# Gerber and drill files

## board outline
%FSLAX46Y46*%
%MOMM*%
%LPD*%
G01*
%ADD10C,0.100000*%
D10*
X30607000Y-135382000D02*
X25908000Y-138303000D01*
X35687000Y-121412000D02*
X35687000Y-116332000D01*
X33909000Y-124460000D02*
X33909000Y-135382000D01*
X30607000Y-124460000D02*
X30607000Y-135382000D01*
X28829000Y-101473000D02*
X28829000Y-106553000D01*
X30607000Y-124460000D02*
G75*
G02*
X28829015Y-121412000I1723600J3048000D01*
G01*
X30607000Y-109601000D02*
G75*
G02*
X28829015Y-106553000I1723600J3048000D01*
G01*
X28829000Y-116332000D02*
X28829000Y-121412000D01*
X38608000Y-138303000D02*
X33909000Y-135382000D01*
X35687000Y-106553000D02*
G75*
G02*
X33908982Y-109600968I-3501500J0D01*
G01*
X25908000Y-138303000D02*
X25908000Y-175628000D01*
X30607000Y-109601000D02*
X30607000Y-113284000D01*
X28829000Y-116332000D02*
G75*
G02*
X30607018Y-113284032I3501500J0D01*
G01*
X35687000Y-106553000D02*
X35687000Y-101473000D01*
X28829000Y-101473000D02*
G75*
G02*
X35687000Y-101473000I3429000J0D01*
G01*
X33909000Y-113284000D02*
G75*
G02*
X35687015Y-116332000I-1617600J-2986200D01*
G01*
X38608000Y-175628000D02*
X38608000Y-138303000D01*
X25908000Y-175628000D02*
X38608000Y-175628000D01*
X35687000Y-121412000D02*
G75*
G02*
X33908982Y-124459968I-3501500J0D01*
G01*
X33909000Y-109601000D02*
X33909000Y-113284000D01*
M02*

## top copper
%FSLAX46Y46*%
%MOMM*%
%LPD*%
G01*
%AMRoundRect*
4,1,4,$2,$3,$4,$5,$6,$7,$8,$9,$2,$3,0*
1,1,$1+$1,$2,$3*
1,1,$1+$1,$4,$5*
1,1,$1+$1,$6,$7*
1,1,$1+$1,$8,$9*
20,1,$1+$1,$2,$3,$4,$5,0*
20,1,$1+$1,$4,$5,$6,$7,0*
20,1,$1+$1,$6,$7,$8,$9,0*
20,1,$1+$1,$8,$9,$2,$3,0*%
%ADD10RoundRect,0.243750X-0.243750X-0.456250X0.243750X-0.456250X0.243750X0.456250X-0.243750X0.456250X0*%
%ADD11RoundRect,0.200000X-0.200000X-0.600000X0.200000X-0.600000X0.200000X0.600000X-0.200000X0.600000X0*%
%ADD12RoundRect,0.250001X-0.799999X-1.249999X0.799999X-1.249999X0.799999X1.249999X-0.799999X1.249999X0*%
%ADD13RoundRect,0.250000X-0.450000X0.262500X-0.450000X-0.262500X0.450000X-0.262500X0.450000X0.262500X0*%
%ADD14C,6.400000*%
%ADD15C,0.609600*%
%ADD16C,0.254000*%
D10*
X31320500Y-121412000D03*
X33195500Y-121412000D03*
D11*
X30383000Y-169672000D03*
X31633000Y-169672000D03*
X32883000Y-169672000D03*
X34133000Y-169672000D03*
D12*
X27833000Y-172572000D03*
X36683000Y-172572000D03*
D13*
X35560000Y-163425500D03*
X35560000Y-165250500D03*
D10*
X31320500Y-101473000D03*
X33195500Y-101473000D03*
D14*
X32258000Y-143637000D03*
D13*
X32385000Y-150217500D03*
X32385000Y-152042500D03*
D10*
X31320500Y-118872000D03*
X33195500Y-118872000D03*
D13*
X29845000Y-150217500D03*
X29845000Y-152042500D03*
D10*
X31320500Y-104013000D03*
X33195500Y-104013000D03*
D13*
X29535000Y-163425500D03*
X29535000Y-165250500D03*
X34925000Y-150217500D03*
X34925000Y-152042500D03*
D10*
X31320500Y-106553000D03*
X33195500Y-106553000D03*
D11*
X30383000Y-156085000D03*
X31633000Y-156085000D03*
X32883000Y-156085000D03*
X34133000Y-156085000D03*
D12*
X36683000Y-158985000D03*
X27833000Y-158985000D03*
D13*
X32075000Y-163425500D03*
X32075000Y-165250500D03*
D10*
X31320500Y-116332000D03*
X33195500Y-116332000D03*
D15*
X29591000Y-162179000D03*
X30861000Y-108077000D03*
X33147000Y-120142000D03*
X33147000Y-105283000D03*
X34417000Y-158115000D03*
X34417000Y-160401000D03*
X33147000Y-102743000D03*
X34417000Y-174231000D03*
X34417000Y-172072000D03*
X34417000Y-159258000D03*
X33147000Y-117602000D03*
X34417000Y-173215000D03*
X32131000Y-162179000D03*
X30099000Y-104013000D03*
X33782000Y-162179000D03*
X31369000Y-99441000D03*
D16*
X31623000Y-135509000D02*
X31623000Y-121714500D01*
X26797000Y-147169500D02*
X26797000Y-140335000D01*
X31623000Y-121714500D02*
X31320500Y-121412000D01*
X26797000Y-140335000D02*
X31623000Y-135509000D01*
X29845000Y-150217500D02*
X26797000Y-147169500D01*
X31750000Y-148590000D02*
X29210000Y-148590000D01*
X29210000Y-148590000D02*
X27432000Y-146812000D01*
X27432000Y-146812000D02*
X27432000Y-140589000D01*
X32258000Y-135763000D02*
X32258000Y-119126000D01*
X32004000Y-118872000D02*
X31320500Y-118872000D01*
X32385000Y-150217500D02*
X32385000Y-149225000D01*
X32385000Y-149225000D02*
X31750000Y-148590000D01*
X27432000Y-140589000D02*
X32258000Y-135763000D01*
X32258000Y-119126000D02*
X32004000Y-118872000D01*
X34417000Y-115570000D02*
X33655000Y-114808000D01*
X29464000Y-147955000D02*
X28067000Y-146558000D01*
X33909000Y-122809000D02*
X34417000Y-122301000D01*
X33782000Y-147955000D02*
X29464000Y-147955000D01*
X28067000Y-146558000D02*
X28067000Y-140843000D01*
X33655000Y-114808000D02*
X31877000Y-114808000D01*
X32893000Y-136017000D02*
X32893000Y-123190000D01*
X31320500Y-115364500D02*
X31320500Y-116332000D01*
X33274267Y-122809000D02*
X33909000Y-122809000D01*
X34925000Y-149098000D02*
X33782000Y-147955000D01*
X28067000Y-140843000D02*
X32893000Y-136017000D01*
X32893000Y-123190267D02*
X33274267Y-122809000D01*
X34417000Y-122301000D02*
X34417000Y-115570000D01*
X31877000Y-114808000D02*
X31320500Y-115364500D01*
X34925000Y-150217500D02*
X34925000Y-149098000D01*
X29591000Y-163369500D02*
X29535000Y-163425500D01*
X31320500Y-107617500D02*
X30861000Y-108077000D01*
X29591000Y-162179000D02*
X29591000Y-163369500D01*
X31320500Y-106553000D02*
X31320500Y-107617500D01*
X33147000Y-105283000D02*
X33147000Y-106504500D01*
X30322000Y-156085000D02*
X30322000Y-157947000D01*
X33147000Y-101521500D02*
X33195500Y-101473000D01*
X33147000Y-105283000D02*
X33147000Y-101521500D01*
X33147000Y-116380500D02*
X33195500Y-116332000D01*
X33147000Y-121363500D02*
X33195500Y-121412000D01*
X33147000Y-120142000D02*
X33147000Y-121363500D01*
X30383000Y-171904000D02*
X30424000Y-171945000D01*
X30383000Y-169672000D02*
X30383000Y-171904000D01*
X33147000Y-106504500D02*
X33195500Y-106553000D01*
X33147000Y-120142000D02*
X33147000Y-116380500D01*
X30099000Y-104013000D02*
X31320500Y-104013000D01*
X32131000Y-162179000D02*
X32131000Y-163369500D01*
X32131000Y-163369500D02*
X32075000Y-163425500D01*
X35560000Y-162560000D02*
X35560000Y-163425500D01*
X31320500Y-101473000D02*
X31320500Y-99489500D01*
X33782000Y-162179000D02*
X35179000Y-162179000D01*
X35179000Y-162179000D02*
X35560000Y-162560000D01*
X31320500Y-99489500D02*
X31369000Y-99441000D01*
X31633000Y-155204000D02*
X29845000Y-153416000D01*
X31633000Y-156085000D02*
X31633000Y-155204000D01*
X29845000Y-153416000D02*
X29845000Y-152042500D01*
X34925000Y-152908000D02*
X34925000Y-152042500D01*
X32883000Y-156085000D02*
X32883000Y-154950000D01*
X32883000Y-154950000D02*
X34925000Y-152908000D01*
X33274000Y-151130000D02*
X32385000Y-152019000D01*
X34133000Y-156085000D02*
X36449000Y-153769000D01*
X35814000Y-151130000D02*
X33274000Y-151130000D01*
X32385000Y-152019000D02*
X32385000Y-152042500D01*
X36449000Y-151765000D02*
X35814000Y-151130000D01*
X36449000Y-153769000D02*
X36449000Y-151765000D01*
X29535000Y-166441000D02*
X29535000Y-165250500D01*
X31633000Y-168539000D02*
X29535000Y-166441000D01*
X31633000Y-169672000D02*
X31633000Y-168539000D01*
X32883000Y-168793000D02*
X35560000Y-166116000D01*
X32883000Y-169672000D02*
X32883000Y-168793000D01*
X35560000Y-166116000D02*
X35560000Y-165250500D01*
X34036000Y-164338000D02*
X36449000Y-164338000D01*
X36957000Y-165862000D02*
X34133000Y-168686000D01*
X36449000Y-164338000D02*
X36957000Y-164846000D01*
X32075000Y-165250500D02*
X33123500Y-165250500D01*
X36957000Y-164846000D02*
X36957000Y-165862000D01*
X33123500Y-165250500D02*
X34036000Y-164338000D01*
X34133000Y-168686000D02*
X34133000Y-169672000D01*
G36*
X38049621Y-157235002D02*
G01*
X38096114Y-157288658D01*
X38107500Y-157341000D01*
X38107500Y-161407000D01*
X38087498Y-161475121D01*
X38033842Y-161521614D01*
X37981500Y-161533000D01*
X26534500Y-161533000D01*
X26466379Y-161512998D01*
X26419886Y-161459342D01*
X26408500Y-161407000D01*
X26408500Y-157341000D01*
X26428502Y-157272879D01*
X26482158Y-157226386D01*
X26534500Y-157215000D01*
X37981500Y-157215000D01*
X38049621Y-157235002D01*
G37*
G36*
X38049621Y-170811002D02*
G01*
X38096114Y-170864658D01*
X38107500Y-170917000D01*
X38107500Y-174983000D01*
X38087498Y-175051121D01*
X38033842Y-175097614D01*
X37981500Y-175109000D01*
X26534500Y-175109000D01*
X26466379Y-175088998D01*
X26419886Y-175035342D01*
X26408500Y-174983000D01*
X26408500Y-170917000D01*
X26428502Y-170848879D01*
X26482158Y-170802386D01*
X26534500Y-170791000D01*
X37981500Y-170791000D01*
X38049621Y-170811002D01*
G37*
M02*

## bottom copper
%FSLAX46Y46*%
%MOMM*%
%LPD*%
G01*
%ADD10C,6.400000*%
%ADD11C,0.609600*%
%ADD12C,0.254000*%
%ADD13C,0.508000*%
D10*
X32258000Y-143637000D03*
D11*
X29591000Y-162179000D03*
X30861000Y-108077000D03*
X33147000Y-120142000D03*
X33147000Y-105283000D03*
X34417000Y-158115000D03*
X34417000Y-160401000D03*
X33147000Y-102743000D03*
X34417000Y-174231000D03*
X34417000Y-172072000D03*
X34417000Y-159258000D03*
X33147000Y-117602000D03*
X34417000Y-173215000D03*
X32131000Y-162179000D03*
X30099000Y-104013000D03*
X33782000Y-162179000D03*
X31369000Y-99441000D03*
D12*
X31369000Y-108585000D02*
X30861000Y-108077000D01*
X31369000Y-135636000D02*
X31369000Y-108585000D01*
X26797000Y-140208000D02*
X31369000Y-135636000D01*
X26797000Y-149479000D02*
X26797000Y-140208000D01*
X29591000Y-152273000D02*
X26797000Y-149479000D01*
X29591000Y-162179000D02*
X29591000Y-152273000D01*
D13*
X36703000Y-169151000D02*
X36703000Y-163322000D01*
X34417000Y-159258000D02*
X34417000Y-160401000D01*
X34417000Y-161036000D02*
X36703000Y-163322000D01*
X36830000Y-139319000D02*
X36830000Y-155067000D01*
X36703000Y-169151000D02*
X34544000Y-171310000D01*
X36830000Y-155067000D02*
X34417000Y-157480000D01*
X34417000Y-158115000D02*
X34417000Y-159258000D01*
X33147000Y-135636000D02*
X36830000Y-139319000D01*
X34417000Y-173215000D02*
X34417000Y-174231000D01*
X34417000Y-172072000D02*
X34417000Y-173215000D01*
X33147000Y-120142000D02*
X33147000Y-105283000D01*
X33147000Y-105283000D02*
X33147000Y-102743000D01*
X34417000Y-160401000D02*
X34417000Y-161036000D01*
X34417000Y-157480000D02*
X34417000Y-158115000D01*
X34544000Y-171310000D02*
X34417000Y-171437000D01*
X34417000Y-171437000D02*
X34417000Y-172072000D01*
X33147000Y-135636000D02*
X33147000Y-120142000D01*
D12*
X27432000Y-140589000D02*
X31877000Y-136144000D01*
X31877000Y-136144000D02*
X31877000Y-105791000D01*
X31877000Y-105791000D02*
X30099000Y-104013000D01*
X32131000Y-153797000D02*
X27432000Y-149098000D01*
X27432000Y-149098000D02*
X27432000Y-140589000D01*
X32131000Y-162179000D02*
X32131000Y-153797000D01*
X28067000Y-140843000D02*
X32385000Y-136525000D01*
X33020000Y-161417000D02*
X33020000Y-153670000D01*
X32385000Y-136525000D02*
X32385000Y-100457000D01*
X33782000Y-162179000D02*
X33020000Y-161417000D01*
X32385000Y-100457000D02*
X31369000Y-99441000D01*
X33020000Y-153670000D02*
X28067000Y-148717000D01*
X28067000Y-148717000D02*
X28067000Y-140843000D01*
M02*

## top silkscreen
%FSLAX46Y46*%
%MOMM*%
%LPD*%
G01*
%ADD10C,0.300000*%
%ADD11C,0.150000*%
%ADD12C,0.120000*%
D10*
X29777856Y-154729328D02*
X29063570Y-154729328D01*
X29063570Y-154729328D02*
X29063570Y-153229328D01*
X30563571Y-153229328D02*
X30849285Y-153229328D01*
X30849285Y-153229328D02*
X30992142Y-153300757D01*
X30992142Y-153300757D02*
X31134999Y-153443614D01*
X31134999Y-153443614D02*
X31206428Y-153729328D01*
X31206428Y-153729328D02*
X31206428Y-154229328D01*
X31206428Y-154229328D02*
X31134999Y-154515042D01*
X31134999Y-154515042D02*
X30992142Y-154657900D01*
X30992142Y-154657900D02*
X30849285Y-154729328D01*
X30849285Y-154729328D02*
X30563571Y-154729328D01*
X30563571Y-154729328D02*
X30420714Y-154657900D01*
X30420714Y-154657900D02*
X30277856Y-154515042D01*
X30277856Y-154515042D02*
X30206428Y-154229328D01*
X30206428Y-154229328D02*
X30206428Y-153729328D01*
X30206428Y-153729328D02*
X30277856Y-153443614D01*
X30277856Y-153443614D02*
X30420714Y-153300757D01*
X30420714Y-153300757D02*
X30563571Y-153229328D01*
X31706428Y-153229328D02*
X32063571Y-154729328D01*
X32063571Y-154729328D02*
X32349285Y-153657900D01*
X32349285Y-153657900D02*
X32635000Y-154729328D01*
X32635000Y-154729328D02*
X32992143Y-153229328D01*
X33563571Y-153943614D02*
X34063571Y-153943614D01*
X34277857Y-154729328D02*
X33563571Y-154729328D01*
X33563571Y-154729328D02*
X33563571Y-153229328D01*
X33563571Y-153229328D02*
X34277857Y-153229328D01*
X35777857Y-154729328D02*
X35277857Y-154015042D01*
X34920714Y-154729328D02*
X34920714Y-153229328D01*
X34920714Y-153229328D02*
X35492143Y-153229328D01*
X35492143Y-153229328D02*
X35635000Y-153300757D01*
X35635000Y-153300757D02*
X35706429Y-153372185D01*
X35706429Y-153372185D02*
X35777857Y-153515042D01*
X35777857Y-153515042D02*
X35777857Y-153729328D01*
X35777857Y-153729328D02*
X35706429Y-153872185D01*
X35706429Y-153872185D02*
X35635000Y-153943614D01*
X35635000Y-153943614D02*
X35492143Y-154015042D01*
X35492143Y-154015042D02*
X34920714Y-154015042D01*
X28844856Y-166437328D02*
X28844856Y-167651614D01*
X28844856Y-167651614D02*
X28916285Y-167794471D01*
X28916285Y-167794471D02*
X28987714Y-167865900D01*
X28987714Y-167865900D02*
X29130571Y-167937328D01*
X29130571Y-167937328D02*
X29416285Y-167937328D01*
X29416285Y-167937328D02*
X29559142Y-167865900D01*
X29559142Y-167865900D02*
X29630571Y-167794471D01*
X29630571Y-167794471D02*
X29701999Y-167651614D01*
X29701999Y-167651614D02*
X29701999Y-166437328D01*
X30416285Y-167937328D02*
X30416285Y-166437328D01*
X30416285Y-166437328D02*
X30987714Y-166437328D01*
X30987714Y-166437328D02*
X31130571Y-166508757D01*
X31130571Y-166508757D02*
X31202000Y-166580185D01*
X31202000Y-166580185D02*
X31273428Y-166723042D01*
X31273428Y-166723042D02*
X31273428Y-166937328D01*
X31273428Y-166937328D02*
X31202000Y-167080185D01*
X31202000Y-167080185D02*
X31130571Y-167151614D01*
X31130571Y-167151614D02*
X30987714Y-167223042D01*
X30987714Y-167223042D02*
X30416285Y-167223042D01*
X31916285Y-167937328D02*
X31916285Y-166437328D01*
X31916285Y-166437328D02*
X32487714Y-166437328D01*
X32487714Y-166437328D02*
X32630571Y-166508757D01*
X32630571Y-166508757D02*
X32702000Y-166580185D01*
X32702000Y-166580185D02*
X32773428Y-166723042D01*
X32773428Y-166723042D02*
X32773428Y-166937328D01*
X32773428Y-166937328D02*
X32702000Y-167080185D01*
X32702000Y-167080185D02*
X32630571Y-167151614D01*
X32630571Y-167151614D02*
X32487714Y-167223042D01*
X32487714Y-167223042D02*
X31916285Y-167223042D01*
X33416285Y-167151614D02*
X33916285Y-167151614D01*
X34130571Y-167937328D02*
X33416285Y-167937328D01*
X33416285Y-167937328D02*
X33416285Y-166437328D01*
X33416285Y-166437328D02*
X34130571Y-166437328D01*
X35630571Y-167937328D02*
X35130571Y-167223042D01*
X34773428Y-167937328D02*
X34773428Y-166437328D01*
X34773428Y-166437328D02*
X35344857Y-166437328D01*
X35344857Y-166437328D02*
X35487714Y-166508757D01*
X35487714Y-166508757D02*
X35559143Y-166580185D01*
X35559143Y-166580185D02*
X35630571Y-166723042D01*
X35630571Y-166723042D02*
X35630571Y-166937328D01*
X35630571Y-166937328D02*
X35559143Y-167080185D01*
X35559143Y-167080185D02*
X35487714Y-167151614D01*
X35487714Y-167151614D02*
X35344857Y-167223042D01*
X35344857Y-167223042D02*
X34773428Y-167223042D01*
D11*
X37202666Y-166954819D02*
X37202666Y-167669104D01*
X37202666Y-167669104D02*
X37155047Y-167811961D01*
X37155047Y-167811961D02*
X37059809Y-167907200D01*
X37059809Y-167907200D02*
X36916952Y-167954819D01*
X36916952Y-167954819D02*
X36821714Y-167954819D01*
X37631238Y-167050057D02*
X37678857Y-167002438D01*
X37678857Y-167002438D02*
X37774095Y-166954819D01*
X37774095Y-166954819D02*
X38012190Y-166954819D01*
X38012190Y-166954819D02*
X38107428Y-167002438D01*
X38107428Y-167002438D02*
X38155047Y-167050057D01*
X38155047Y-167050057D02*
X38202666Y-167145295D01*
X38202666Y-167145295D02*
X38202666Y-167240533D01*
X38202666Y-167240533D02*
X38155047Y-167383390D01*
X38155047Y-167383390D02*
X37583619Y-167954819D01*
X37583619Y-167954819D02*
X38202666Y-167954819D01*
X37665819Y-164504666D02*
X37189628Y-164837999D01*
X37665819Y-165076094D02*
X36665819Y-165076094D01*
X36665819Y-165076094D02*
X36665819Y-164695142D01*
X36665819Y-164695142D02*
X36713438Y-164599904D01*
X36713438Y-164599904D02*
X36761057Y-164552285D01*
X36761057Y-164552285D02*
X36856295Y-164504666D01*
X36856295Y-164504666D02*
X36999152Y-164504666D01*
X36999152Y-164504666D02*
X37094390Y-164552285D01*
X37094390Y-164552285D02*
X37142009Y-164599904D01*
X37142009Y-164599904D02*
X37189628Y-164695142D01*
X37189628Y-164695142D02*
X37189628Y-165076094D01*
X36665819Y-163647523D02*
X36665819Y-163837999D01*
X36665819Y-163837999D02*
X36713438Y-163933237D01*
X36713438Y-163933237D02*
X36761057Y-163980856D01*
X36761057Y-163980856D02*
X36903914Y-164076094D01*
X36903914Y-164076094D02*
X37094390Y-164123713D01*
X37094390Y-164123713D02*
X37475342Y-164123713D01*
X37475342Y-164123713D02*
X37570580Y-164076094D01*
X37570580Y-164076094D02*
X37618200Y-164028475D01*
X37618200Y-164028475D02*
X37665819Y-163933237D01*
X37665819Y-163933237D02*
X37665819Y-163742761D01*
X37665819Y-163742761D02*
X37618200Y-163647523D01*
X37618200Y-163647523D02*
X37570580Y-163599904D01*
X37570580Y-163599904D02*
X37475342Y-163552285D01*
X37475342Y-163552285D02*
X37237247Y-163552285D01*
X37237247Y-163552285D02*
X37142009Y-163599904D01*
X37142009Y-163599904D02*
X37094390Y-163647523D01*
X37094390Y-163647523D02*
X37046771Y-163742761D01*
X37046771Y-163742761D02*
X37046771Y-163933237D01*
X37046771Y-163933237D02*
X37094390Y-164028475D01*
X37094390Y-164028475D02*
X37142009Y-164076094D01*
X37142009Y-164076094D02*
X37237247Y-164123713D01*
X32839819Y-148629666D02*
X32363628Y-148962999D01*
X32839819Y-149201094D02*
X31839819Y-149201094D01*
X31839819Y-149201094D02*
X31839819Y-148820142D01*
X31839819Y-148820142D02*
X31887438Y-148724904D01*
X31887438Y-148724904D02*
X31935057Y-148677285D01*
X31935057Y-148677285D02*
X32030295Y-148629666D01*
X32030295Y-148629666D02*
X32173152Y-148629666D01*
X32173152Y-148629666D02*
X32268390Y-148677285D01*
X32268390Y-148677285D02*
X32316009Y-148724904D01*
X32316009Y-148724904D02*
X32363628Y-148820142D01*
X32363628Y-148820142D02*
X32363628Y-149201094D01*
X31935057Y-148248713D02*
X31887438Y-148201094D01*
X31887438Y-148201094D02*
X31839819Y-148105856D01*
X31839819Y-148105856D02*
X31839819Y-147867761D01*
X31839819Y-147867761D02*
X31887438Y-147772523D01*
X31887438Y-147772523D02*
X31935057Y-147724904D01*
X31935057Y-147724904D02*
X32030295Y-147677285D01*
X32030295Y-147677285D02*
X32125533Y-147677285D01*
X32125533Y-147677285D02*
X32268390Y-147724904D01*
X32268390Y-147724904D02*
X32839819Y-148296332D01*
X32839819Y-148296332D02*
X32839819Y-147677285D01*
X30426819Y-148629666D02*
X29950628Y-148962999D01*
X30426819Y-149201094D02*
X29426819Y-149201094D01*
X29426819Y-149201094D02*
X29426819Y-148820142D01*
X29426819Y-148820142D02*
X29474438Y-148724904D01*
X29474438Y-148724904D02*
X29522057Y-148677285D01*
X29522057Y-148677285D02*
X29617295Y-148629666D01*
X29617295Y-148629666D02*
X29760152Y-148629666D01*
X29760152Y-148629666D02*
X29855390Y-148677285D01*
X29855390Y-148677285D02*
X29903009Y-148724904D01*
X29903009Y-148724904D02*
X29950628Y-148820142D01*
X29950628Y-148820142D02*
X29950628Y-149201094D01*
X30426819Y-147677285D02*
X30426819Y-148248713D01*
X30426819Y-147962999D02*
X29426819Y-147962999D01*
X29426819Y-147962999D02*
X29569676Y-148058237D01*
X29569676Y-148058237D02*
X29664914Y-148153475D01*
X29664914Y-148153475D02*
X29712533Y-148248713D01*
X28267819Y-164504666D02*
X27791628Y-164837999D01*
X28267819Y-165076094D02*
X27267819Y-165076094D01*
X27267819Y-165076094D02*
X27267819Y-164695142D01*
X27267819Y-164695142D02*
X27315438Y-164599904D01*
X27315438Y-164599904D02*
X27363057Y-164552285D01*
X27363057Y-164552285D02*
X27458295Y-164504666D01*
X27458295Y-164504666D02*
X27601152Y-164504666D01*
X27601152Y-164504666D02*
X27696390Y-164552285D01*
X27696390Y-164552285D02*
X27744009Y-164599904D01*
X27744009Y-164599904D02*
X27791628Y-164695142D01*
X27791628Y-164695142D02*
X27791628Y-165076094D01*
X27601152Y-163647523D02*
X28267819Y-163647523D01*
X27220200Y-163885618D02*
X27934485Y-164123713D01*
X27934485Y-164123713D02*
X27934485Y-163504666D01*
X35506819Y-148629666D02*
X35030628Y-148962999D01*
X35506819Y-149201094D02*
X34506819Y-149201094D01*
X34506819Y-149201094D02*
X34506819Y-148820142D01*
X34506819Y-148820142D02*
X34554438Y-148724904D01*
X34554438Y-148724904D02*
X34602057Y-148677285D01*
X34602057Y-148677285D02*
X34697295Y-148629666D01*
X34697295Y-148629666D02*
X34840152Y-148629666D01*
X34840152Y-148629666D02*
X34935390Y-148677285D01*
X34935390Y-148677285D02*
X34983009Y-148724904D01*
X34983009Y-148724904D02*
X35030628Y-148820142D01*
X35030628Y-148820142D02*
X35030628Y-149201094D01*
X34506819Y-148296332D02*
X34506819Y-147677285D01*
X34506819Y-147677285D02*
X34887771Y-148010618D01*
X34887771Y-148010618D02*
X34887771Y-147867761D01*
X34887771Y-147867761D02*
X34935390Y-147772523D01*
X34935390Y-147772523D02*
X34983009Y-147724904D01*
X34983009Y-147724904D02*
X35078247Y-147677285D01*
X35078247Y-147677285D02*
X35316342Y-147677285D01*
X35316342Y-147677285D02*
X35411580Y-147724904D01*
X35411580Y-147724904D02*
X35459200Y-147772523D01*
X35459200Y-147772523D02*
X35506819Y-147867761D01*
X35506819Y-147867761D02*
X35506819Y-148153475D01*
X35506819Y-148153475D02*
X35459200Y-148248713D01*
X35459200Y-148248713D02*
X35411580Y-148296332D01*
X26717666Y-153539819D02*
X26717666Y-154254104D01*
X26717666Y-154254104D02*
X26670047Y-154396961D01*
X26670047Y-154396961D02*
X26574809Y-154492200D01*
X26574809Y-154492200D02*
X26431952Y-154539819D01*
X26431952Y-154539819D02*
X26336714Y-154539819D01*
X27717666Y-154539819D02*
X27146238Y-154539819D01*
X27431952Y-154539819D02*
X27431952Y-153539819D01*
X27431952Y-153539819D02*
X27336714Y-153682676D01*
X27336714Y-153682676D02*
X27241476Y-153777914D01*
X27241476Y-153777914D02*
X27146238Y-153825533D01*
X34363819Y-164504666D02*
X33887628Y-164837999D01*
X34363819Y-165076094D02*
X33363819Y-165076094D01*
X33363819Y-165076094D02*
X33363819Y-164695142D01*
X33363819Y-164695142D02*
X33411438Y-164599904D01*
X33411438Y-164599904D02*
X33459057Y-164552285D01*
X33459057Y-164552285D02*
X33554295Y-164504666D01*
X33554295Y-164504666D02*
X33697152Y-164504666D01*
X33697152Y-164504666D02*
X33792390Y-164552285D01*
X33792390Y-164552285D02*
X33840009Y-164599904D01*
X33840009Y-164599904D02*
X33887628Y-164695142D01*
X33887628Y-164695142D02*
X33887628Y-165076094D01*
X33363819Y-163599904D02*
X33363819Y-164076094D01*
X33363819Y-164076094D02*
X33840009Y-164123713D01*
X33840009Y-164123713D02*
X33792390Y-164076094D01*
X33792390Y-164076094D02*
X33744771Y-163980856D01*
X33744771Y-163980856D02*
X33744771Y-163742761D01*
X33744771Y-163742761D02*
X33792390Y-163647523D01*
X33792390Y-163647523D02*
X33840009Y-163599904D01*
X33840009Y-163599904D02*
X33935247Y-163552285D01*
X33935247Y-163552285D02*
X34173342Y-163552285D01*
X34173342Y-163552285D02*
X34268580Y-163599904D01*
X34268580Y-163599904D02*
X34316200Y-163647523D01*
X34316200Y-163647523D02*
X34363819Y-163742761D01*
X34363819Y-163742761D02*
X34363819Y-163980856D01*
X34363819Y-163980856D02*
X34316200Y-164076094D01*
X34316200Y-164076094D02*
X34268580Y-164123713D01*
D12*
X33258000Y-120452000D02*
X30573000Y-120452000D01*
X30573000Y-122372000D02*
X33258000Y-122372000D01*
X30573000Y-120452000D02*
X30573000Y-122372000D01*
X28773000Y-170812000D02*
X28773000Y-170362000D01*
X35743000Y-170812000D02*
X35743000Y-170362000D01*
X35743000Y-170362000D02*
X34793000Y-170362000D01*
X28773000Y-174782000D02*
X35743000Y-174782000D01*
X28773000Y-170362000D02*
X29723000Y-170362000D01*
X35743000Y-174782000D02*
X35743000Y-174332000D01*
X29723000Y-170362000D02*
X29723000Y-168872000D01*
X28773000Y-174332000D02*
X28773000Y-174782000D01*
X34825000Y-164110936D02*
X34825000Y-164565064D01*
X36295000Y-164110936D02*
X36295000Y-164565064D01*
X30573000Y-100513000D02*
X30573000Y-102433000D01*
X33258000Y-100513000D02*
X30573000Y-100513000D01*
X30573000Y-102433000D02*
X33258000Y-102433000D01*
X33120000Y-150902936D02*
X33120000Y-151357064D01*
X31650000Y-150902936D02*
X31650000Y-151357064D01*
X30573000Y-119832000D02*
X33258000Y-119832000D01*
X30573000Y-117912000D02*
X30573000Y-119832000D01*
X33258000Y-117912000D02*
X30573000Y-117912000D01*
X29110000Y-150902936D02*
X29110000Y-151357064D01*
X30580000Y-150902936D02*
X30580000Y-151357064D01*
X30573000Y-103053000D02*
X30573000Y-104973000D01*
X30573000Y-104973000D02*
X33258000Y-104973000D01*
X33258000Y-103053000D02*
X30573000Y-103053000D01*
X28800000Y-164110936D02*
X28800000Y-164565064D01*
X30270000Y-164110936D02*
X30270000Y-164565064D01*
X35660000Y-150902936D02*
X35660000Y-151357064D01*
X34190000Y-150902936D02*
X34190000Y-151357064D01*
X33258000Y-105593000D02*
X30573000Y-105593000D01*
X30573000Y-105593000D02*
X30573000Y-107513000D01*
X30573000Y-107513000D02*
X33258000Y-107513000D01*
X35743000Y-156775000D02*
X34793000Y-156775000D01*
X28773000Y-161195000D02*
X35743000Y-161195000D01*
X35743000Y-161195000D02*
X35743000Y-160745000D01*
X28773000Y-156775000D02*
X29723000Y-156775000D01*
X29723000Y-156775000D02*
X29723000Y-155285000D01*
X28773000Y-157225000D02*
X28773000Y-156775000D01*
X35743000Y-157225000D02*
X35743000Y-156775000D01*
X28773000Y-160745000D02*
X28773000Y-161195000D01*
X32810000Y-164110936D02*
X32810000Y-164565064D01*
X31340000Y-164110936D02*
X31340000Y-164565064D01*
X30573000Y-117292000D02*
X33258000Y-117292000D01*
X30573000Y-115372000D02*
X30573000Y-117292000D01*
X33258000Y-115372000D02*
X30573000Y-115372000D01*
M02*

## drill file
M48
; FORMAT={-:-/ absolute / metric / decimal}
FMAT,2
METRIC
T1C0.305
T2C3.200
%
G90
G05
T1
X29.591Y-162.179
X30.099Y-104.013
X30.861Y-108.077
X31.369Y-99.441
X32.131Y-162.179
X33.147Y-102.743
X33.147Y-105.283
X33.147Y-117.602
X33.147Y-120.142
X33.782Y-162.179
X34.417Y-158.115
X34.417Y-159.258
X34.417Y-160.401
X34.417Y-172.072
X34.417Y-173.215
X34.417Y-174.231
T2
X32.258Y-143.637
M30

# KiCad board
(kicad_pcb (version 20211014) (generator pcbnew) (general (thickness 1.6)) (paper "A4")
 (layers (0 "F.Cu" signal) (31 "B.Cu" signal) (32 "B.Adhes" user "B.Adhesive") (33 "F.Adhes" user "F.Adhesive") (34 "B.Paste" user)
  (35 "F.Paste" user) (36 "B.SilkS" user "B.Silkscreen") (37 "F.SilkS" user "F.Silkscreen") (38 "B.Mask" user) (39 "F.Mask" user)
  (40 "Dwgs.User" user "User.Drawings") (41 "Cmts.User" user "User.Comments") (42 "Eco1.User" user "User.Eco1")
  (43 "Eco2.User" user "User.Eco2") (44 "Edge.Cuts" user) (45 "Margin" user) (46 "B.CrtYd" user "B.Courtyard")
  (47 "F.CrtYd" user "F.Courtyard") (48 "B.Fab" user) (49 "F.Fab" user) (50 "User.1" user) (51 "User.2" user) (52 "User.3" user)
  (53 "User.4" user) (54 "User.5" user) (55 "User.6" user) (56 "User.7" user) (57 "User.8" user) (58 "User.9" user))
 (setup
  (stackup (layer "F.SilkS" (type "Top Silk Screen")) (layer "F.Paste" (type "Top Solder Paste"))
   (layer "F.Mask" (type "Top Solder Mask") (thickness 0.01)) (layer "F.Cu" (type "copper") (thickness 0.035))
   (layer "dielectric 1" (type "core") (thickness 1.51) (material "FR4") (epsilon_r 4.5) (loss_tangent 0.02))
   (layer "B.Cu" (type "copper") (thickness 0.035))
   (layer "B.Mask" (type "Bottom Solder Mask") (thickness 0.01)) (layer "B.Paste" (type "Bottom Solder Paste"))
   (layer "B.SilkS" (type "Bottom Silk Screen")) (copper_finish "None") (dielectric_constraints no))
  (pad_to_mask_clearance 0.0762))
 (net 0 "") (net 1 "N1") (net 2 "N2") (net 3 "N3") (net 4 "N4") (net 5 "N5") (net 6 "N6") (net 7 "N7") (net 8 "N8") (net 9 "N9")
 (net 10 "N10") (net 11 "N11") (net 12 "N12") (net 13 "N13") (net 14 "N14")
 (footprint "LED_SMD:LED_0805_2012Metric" (layer "F.Cu") (at 32.258 121.412)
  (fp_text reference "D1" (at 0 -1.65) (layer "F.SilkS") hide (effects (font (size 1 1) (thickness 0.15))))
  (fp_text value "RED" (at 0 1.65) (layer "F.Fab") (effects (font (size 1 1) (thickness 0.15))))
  (fp_line (start 1 -0.96) (end -1.685 -0.96) (layer "F.SilkS") (width 0.12))
  (fp_line (start -1.685 0.96) (end 1 0.96) (layer "F.SilkS") (width 0.12))
  (fp_line (start -1.685 -0.96) (end -1.685 0.96) (layer "F.SilkS") (width 0.12))
  (pad "1" smd roundrect (at -0.9375 0) (size 0.975 1.4) (layers "F.Cu" "F.Paste" "F.Mask") (roundrect_rratio 0.25) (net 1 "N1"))
  (pad "2" smd roundrect (at 0.9375 0) (size 0.975 1.4) (layers "F.Cu" "F.Paste" "F.Mask") (roundrect_rratio 0.25) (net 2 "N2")))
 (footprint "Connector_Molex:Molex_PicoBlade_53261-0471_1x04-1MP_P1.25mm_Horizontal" (layer "F.Cu") (at 32.258 172.072)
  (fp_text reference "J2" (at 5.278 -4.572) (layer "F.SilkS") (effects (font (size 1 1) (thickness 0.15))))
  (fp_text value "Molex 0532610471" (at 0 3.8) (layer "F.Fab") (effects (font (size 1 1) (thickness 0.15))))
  (fp_line (start -3.485 -1.26) (end -3.485 -1.71) (layer "F.SilkS") (width 0.12))
  (fp_line (start 3.485 -1.26) (end 3.485 -1.71) (layer "F.SilkS") (width 0.12))
  (fp_line (start 3.485 -1.71) (end 2.535 -1.71) (layer "F.SilkS") (width 0.12))
  (fp_line (start -3.485 2.71) (end 3.485 2.71) (layer "F.SilkS") (width 0.12))
  (fp_line (start -3.485 -1.71) (end -2.535 -1.71) (layer "F.SilkS") (width 0.12))
  (fp_line (start 3.485 2.71) (end 3.485 2.26) (layer "F.SilkS") (width 0.12))
  (fp_line (start -2.535 -1.71) (end -2.535 -3.2) (layer "F.SilkS") (width 0.12))
  (fp_line (start -3.485 2.26) (end -3.485 2.71) (layer "F.SilkS") (width 0.12))
  (pad "1" smd roundrect (at -1.875 -2.4) (size 0.8 1.6) (layers "F.Cu" "F.Paste" "F.Mask") (roundrect_rratio 0.25) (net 2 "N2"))
  (pad "2" smd roundrect (at -0.625 -2.4) (size 0.8 1.6) (layers "F.Cu" "F.Paste" "F.Mask") (roundrect_rratio 0.25) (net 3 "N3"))
  (pad "3" smd roundrect (at 0.625 -2.4) (size 0.8 1.6) (layers "F.Cu" "F.Paste" "F.Mask") (roundrect_rratio 0.25) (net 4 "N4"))
  (pad "4" smd roundrect (at 1.875 -2.4) (size 0.8 1.6) (layers "F.Cu" "F.Paste" "F.Mask") (roundrect_rratio 0.25) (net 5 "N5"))
  (pad "MP" smd roundrect (at -4.425 0.5) (size 2.1 3) (layers "F.Cu" "F.Paste" "F.Mask") (roundrect_rratio 0.119048) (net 2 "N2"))
  (pad "MP" smd roundrect (at 4.425 0.5) (size 2.1 3) (layers "F.Cu" "F.Paste" "F.Mask") (roundrect_rratio 0.119048) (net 2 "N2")))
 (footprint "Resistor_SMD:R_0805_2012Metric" (layer "F.Cu") (at 35.56 164.338 -90)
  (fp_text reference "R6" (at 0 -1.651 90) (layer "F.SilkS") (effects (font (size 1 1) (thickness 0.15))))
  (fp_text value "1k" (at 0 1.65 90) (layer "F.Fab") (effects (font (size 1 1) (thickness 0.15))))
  (fp_line (start -0.227064 0.735) (end 0.227064 0.735) (layer "F.SilkS") (width 0.12))
  (fp_line (start -0.227064 -0.735) (end 0.227064 -0.735) (layer "F.SilkS") (width 0.12))
  (pad "1" smd roundrect (at -0.9125 0 270) (size 1.025 1.4) (layers "F.Cu" "F.Paste" "F.Mask") (roundrect_rratio 0.243902) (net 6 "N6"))
  (pad "2" smd roundrect (at 0.9125 0 270) (size 1.025 1.4) (layers "F.Cu" "F.Paste" "F.Mask") (roundrect_rratio 0.243902) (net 4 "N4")))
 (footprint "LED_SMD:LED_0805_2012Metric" (layer "F.Cu") (at 32.258 101.473)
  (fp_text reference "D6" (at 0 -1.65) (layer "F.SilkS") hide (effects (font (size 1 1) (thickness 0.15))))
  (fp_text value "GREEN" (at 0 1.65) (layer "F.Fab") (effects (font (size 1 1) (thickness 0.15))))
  (fp_line (start -1.685 -0.96) (end -1.685 0.96) (layer "F.SilkS") (width 0.12))
  (fp_line (start 1 -0.96) (end -1.685 -0.96) (layer "F.SilkS") (width 0.12))
  (fp_line (start -1.685 0.96) (end 1 0.96) (layer "F.SilkS") (width 0.12))
  (pad "1" smd roundrect (at -0.9375 0) (size 0.975 1.4) (layers "F.Cu" "F.Paste" "F.Mask") (roundrect_rratio 0.25) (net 6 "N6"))
  (pad "2" smd roundrect (at 0.9375 0) (size 0.975 1.4) (layers "F.Cu" "F.Paste" "F.Mask") (roundrect_rratio 0.25) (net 2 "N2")))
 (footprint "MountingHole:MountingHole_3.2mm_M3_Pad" (layer "F.Cu") (at 32.258 143.637) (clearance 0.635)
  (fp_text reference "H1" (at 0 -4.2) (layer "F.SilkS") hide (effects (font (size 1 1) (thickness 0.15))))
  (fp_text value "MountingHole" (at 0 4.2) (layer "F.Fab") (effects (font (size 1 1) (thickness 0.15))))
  (pad "1" thru_hole circle (at 0 0) (size 6.4 6.4) (drill 3.2) (layers *.Cu *.Mask) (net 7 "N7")))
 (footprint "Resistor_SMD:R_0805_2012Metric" (layer "F.Cu") (at 32.385 151.13 -90)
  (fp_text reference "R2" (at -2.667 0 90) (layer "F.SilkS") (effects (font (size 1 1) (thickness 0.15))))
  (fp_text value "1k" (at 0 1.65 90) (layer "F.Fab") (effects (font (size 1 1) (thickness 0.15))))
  (fp_line (start -0.227064 -0.735) (end 0.227064 -0.735) (layer "F.SilkS") (width 0.12))
  (fp_line (start -0.227064 0.735) (end 0.227064 0.735) (layer "F.SilkS") (width 0.12))
  (pad "1" smd roundrect (at -0.9125 0 270) (size 1.025 1.4) (layers "F.Cu" "F.Paste" "F.Mask") (roundrect_rratio 0.243902) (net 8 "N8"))
  (pad "2" smd roundrect (at 0.9125 0 270) (size 1.025 1.4) (layers "F.Cu" "F.Paste" "F.Mask") (roundrect_rratio 0.243902) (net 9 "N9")))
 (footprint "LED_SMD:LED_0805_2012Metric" (layer "F.Cu") (at 32.258 118.872)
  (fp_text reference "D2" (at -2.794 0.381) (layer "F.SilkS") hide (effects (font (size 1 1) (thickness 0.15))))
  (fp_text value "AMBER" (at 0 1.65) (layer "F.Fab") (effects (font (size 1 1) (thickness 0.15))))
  (fp_line (start -1.685 0.96) (end 1 0.96) (layer "F.SilkS") (width 0.12))
  (fp_line (start -1.685 -0.96) (end -1.685 0.96) (layer "F.SilkS") (width 0.12))
  (fp_line (start 1 -0.96) (end -1.685 -0.96) (layer "F.SilkS") (width 0.12))
  (pad "1" smd roundrect (at -0.9375 0) (size 0.975 1.4) (layers "F.Cu" "F.Paste" "F.Mask") (roundrect_rratio 0.25) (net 8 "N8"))
  (pad "2" smd roundrect (at 0.9375 0) (size 0.975 1.4) (layers "F.Cu" "F.Paste" "F.Mask") (roundrect_rratio 0.25) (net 2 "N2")))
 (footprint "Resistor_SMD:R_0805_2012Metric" (layer "F.Cu") (at 29.845 151.13 -90)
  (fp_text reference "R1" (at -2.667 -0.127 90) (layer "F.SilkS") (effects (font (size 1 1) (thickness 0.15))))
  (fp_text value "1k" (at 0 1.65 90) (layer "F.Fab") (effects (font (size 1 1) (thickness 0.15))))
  (fp_line (start -0.227064 0.735) (end 0.227064 0.735) (layer "F.SilkS") (width 0.12))
  (fp_line (start -0.227064 -0.735) (end 0.227064 -0.735) (layer "F.SilkS") (width 0.12))
  (pad "1" smd roundrect (at -0.9125 0 270) (size 1.025 1.4) (layers "F.Cu" "F.Paste" "F.Mask") (roundrect_rratio 0.243902) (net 1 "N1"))
  (pad "2" smd roundrect (at 0.9125 0 270) (size 1.025 1.4) (layers "F.Cu" "F.Paste" "F.Mask") (roundrect_rratio 0.243902) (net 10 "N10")))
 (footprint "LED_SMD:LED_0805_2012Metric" (layer "F.Cu") (at 32.258 104.013)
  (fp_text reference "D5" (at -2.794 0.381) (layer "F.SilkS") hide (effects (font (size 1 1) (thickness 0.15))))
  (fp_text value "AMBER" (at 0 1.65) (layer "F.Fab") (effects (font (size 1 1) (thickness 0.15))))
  (fp_line (start -1.685 -0.96) (end -1.685 0.96) (layer "F.SilkS") (width 0.12))
  (fp_line (start -1.685 0.96) (end 1 0.96) (layer "F.SilkS") (width 0.12))
  (fp_line (start 1 -0.96) (end -1.685 -0.96) (layer "F.SilkS") (width 0.12))
  (pad "1" smd roundrect (at -0.9375 0) (size 0.975 1.4) (layers "F.Cu" "F.Paste" "F.Mask") (roundrect_rratio 0.25) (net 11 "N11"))
  (pad "2" smd roundrect (at 0.9375 0) (size 0.975 1.4) (layers "F.Cu" "F.Paste" "F.Mask") (roundrect_rratio 0.25) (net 2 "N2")))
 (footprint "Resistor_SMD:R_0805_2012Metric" (layer "F.Cu") (at 29.535 164.338 -90)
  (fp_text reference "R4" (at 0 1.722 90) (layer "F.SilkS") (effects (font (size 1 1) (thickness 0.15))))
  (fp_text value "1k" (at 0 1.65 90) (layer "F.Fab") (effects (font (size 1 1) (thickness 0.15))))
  (fp_line (start -0.227064 0.735) (end 0.227064 0.735) (layer "F.SilkS") (width 0.12))
  (fp_line (start -0.227064 -0.735) (end 0.227064 -0.735) (layer "F.SilkS") (width 0.12))
  (pad "1" smd roundrect (at -0.9125 0 270) (size 1.025 1.4) (layers "F.Cu" "F.Paste" "F.Mask") (roundrect_rratio 0.243902) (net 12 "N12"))
  (pad "2" smd roundrect (at 0.9125 0 270) (size 1.025 1.4) (layers "F.Cu" "F.Paste" "F.Mask") (roundrect_rratio 0.243902) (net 3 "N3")))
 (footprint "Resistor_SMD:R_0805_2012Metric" (layer "F.Cu") (at 34.925 151.13 -90)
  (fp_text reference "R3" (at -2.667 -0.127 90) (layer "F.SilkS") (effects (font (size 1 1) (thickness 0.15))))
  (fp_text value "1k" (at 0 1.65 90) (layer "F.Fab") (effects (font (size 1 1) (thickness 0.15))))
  (fp_line (start -0.227064 -0.735) (end 0.227064 -0.735) (layer "F.SilkS") (width 0.12))
  (fp_line (start -0.227064 0.735) (end 0.227064 0.735) (layer "F.SilkS") (width 0.12))
  (pad "1" smd roundrect (at -0.9125 0 270) (size 1.025 1.4) (layers "F.Cu" "F.Paste" "F.Mask") (roundrect_rratio 0.243902) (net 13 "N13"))
  (pad "2" smd roundrect (at 0.9125 0 270) (size 1.025 1.4) (layers "F.Cu" "F.Paste" "F.Mask") (roundrect_rratio 0.243902) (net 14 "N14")))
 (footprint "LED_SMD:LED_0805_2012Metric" (layer "F.Cu") (at 32.258 106.553)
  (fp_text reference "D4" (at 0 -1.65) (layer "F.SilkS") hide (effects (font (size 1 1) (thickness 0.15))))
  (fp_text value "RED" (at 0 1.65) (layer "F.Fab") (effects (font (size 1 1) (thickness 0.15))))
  (fp_line (start 1 -0.96) (end -1.685 -0.96) (layer "F.SilkS") (width 0.12))
  (fp_line (start -1.685 -0.96) (end -1.685 0.96) (layer "F.SilkS") (width 0.12))
  (fp_line (start -1.685 0.96) (end 1 0.96) (layer "F.SilkS") (width 0.12))
  (pad "1" smd roundrect (at -0.9375 0) (size 0.975 1.4) (layers "F.Cu" "F.Paste" "F.Mask") (roundrect_rratio 0.25) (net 12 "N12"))
  (pad "2" smd roundrect (at 0.9375 0) (size 0.975 1.4) (layers "F.Cu" "F.Paste" "F.Mask") (roundrect_rratio 0.25) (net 2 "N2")))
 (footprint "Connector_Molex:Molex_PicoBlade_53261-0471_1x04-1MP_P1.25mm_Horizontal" (layer "F.Cu") (at 32.258 158.485)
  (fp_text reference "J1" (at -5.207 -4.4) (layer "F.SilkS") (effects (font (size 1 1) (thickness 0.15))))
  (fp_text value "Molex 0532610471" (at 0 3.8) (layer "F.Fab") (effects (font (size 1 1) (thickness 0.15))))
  (fp_line (start 3.485 -1.71) (end 2.535 -1.71) (layer "F.SilkS") (width 0.12))
  (fp_line (start -3.485 2.71) (end 3.485 2.71) (layer "F.SilkS") (width 0.12))
  (fp_line (start 3.485 2.71) (end 3.485 2.26) (layer "F.SilkS") (width 0.12))
  (fp_line (start -3.485 -1.71) (end -2.535 -1.71) (layer "F.SilkS") (width 0.12))
  (fp_line (start -2.535 -1.71) (end -2.535 -3.2) (layer "F.SilkS") (width 0.12))
  (fp_line (start -3.485 -1.26) (end -3.485 -1.71) (layer "F.SilkS") (width 0.12))
  (fp_line (start 3.485 -1.26) (end 3.485 -1.71) (layer "F.SilkS") (width 0.12))
  (fp_line (start -3.485 2.26) (end -3.485 2.71) (layer "F.SilkS") (width 0.12))
  (pad "1" smd roundrect (at -1.875 -2.4) (size 0.8 1.6) (layers "F.Cu" "F.Paste" "F.Mask") (roundrect_rratio 0.25) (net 2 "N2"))
  (pad "2" smd roundrect (at -0.625 -2.4) (size 0.8 1.6) (layers "F.Cu" "F.Paste" "F.Mask") (roundrect_rratio 0.25) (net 10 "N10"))
  (pad "3" smd roundrect (at 0.625 -2.4) (size 0.8 1.6) (layers "F.Cu" "F.Paste" "F.Mask") (roundrect_rratio 0.25) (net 14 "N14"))
  (pad "4" smd roundrect (at 1.875 -2.4) (size 0.8 1.6) (layers "F.Cu" "F.Paste" "F.Mask") (roundrect_rratio 0.25) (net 9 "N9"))
  (pad "MP" smd roundrect (at 4.425 0.5) (size 2.1 3) (layers "F.Cu" "F.Paste" "F.Mask") (roundrect_rratio 0.119048) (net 2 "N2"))
  (pad "MP" smd roundrect (at -4.425 0.5) (size 2.1 3) (layers "F.Cu" "F.Paste" "F.Mask") (roundrect_rratio 0.119048) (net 2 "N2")))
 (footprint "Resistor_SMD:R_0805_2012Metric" (layer "F.Cu") (at 32.075 164.338 -90)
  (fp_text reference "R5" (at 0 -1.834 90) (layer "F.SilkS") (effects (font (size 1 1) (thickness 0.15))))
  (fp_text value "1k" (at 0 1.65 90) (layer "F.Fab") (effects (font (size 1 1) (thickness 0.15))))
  (fp_line (start -0.227064 -0.735) (end 0.227064 -0.735) (layer "F.SilkS") (width 0.12))
  (fp_line (start -0.227064 0.735) (end 0.227064 0.735) (layer "F.SilkS") (width 0.12))
  (pad "1" smd roundrect (at -0.9125 0 270) (size 1.025 1.4) (layers "F.Cu" "F.Paste" "F.Mask") (roundrect_rratio 0.243902) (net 11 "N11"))
  (pad "2" smd roundrect (at 0.9125 0 270) (size 1.025 1.4) (layers "F.Cu" "F.Paste" "F.Mask") (roundrect_rratio 0.243902) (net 5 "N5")))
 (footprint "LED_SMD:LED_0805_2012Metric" (layer "F.Cu") (at 32.258 116.332)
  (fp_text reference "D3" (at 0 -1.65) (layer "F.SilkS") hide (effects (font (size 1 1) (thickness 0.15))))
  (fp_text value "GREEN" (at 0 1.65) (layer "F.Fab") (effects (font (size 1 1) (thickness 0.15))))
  (fp_line (start -1.685 0.96) (end 1 0.96) (layer "F.SilkS") (width 0.12))
  (fp_line (start -1.685 -0.96) (end -1.685 0.96) (layer "F.SilkS") (width 0.12))
  (fp_line (start 1 -0.96) (end -1.685 -0.96) (layer "F.SilkS") (width 0.12))
  (pad "1" smd roundrect (at -0.9375 0) (size 0.975 1.4) (layers "F.Cu" "F.Paste" "F.Mask") (roundrect_rratio 0.25) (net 13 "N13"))
  (pad "2" smd roundrect (at 0.9375 0) (size 0.975 1.4) (layers "F.Cu" "F.Paste" "F.Mask") (roundrect_rratio 0.25) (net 2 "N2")))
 (gr_line (start 30.607 135.382) (end 25.908 138.303) (layer "Edge.Cuts") (width 0.1))
 (gr_line (start 35.687 121.412) (end 35.687 116.332) (layer "Edge.Cuts") (width 0.1))
 (gr_line (start 33.909 124.46) (end 33.909 135.382) (layer "Edge.Cuts") (width 0.1))
 (gr_line (start 30.607 124.46) (end 30.607 135.382) (layer "Edge.Cuts") (width 0.1))
 (gr_line (start 28.829 101.473) (end 28.829 106.553) (layer "Edge.Cuts") (width 0.1))
 (gr_arc (start 30.607 124.46) (mid 29.305998 123.176337) (end 28.829 121.412) (layer "Edge.Cuts") (width 0.1))
 (gr_arc (start 30.607 109.601) (mid 29.305998 108.317337) (end 28.829 106.553) (layer "Edge.Cuts") (width 0.1))
 (gr_line (start 28.829 116.332) (end 28.829 121.412) (layer "Edge.Cuts") (width 0.1))
 (gr_line (start 38.608 138.303) (end 33.909 135.382) (layer "Edge.Cuts") (width 0.1))
 (gr_arc (start 35.687 106.553) (mid 35.210014 108.317344) (end 33.909 109.601) (layer "Edge.Cuts") (width 0.1))
 (gr_line (start 25.908 138.303) (end 25.908 175.628) (layer "Edge.Cuts") (width 0.1))
 (gr_line (start 30.607 109.601) (end 30.607 113.284) (layer "Edge.Cuts") (width 0.1))
 (gr_arc (start 28.829 116.332) (mid 29.305986 114.567656) (end 30.607 113.284) (layer "Edge.Cuts") (width 0.1))
 (gr_line (start 35.687 106.553) (end 35.687 101.473) (layer "Edge.Cuts") (width 0.1))
 (gr_arc (start 28.829 101.473) (mid 32.258 98.044) (end 35.687 101.473) (layer "Edge.Cuts") (width 0.1))
 (gr_arc (start 33.909 113.284) (mid 35.224938 114.558949) (end 35.687 116.332) (layer "Edge.Cuts") (width 0.1))
 (gr_line (start 38.608 175.628) (end 38.608 138.303) (layer "Edge.Cuts") (width 0.1))
 (gr_line (start 25.908 175.628) (end 38.608 175.628) (layer "Edge.Cuts") (width 0.1))
 (gr_arc (start 35.687 121.412) (mid 35.210014 123.176344) (end 33.909 124.46) (layer "Edge.Cuts") (width 0.1))
 (gr_line (start 33.909 109.601) (end 33.909 113.284) (layer "Edge.Cuts") (width 0.1))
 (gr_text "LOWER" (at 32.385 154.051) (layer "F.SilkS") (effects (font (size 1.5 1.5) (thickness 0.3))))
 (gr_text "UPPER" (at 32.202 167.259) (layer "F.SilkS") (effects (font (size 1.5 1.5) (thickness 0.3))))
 (segment (start 31.623 135.509) (end 31.623 121.7145) (width 0.254) (layer "F.Cu") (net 1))
 (segment (start 26.797 147.1695) (end 26.797 140.335) (width 0.254) (layer "F.Cu") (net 1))
 (segment (start 31.623 121.7145) (end 31.3205 121.412) (width 0.254) (layer "F.Cu") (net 1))
 (segment (start 26.797 140.335) (end 31.623 135.509) (width 0.254) (layer "F.Cu") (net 1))
 (segment (start 29.845 150.2175) (end 26.797 147.1695) (width 0.254) (layer "F.Cu") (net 1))
 (segment (start 31.75 148.59) (end 29.21 148.59) (width 0.254) (layer "F.Cu") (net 8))
 (segment (start 29.21 148.59) (end 27.432 146.812) (width 0.254) (layer "F.Cu") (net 8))
 (segment (start 27.432 146.812) (end 27.432 140.589) (width 0.254) (layer "F.Cu") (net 8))
 (segment (start 32.258 135.763) (end 32.258 119.126) (width 0.254) (layer "F.Cu") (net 8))
 (segment (start 32.004 118.872) (end 31.3205 118.872) (width 0.254) (layer "F.Cu") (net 8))
 (segment (start 32.385 150.2175) (end 32.385 149.225) (width 0.254) (layer "F.Cu") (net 8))
 (segment (start 32.385 149.225) (end 31.75 148.59) (width 0.254) (layer "F.Cu") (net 8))
 (segment (start 27.432 140.589) (end 32.258 135.763) (width 0.254) (layer "F.Cu") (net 8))
 (segment (start 32.258 119.126) (end 32.004 118.872) (width 0.254) (layer "F.Cu") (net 8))
 (segment (start 34.417 115.57) (end 33.655 114.808) (width 0.254) (layer "F.Cu") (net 13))
 (segment (start 29.464 147.955) (end 28.067 146.558) (width 0.254) (layer "F.Cu") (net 13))
 (segment (start 33.909 122.809) (end 34.417 122.301) (width 0.254) (layer "F.Cu") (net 13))
 (segment (start 33.782 147.955) (end 29.464 147.955) (width 0.254) (layer "F.Cu") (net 13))
 (segment (start 28.067 146.558) (end 28.067 140.843) (width 0.254) (layer "F.Cu") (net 13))
 (segment (start 33.655 114.808) (end 31.877 114.808) (width 0.254) (layer "F.Cu") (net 13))
 (segment (start 32.893 136.017) (end 32.893 123.19) (width 0.254) (layer "F.Cu") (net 13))
 (segment (start 31.3205 115.3645) (end 31.3205 116.332) (width 0.254) (layer "F.Cu") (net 13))
 (segment (start 33.274267 122.809) (end 33.909 122.809) (width 0.254) (layer "F.Cu") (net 13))
 (segment (start 34.925 149.098) (end 33.782 147.955) (width 0.254) (layer "F.Cu") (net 13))
 (segment (start 28.067 140.843) (end 32.893 136.017) (width 0.254) (layer "F.Cu") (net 13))
 (segment (start 32.893 123.190267) (end 33.274267 122.809) (width 0.254) (layer "F.Cu") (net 13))
 (segment (start 34.417 122.301) (end 34.417 115.57) (width 0.254) (layer "F.Cu") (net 13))
 (segment (start 31.877 114.808) (end 31.3205 115.3645) (width 0.254) (layer "F.Cu") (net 13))
 (segment (start 34.925 150.2175) (end 34.925 149.098) (width 0.254) (layer "F.Cu") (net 13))
 (segment (start 29.591 163.3695) (end 29.535 163.4255) (width 0.254) (layer "F.Cu") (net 12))
 (segment (start 31.3205 107.6175) (end 30.861 108.077) (width 0.254) (layer "F.Cu") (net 12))
 (segment (start 29.591 162.179) (end 29.591 163.3695) (width 0.254) (layer "F.Cu") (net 12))
 (segment (start 31.3205 106.553) (end 31.3205 107.6175) (width 0.254) (layer "F.Cu") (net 12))
 (via (at 29.591 162.179) (size 0.6096) (drill 0.3048) (layers "F.Cu" "B.Cu") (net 12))
 (via (at 30.861 108.077) (size 0.6096) (drill 0.3048) (layers "F.Cu" "B.Cu") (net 12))
 (segment (start 31.369 108.585) (end 30.861 108.077) (width 0.254) (layer "B.Cu") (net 12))
 (segment (start 31.369 135.636) (end 31.369 108.585) (width 0.254) (layer "B.Cu") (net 12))
 (segment (start 26.797 140.208) (end 31.369 135.636) (width 0.254) (layer "B.Cu") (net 12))
 (segment (start 26.797 149.479) (end 26.797 140.208) (width 0.254) (layer "B.Cu") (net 12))
 (segment (start 29.591 152.273) (end 26.797 149.479) (width 0.254) (layer "B.Cu") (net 12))
 (segment (start 29.591 162.179) (end 29.591 152.273) (width 0.254) (layer "B.Cu") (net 12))
 (segment (start 33.147 105.283) (end 33.147 106.5045) (width 0.254) (layer "F.Cu") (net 2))
 (segment (start 30.322 156.085) (end 30.322 157.947) (width 0.254) (layer "F.Cu") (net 2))
 (segment (start 33.147 101.5215) (end 33.1955 101.473) (width 0.254) (layer "F.Cu") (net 2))
 (segment (start 33.147 105.283) (end 33.147 101.5215) (width 0.254) (layer "F.Cu") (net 2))
 (segment (start 33.147 116.3805) (end 33.1955 116.332) (width 0.254) (layer "F.Cu") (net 2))
 (segment (start 33.147 121.3635) (end 33.1955 121.412) (width 0.254) (layer "F.Cu") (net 2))
 (segment (start 33.147 120.142) (end 33.147 121.3635) (width 0.254) (layer "F.Cu") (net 2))
 (segment (start 30.383 171.904) (end 30.424 171.945) (width 0.254) (layer "F.Cu") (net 2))
 (segment (start 30.383 169.672) (end 30.383 171.904) (width 0.254) (layer "F.Cu") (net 2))
 (segment (start 33.147 106.5045) (end 33.1955 106.553) (width 0.254) (layer "F.Cu") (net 2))
 (segment (start 33.147 120.142) (end 33.147 116.3805) (width 0.254) (layer "F.Cu") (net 2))
 (via (at 33.147 120.142) (size 0.6096) (drill 0.3048) (layers "F.Cu" "B.Cu") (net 2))
 (via (at 33.147 105.283) (size 0.6096) (drill 0.3048) (layers "F.Cu" "B.Cu") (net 2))
 (via (at 34.417 158.115) (size 0.6096) (drill 0.3048) (layers "F.Cu" "B.Cu") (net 2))
 (via (at 34.417 160.401) (size 0.6096) (drill 0.3048) (layers "F.Cu" "B.Cu") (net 2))
 (via (at 33.147 102.743) (size 0.6096) (drill 0.3048) (layers "F.Cu" "B.Cu") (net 2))
 (via (at 34.417 174.231) (size 0.6096) (drill 0.3048) (layers "F.Cu" "B.Cu") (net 2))
 (via (at 34.417 172.072) (size 0.6096) (drill 0.3048) (layers "F.Cu" "B.Cu") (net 2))
 (via (at 34.417 159.258) (size 0.6096) (drill 0.3048) (layers "F.Cu" "B.Cu") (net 2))
 (via (at 33.147 117.602) (size 0.6096) (drill 0.3048) (layers "F.Cu" "B.Cu") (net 2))
 (via (at 34.417 173.215) (size 0.6096) (drill 0.3048) (layers "F.Cu" "B.Cu") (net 2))
 (segment (start 36.703 169.151) (end 36.703 163.322) (width 0.508) (layer "B.Cu") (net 2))
 (segment (start 34.417 159.258) (end 34.417 160.401) (width 0.508) (layer "B.Cu") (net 2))
 (segment (start 34.417 161.036) (end 36.703 163.322) (width 0.508) (layer "B.Cu") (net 2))
 (segment (start 36.83 139.319) (end 36.83 155.067) (width 0.508) (layer "B.Cu") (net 2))
 (segment (start 36.703 169.151) (end 34.544 171.31) (width 0.508) (layer "B.Cu") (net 2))
 (segment (start 36.83 155.067) (end 34.417 157.48) (width 0.508) (layer "B.Cu") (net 2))
 (segment (start 34.417 158.115) (end 34.417 159.258) (width 0.508) (layer "B.Cu") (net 2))
 (segment (start 33.147 135.636) (end 36.83 139.319) (width 0.508) (layer "B.Cu") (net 2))
 (segment (start 34.417 173.215) (end 34.417 174.231) (width 0.508) (layer "B.Cu") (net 2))
 (segment (start 34.417 172.072) (end 34.417 173.215) (width 0.508) (layer "B.Cu") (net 2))
 (segment (start 33.147 120.142) (end 33.147 105.283) (width 0.508) (layer "B.Cu") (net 2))
 (segment (start 33.147 105.283) (end 33.147 102.743) (width 0.508) (layer "B.Cu") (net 2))
 (segment (start 34.417 160.401) (end 34.417 161.036) (width 0.508) (layer "B.Cu") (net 2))
 (segment (start 34.417 157.48) (end 34.417 158.115) (width 0.508) (layer "B.Cu") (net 2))
 (segment (start 34.544 171.31) (end 34.417 171.437) (width 0.508) (layer "B.Cu") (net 2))
 (segment (start 34.417 171.437) (end 34.417 172.072) (width 0.508) (layer "B.Cu") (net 2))
 (segment (start 33.147 135.636) (end 33.147 120.142) (width 0.508) (layer "B.Cu") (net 2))
 (segment (start 30.099 104.013) (end 31.3205 104.013) (width 0.254) (layer "F.Cu") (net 11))
 (segment (start 32.131 162.179) (end 32.131 163.3695) (width 0.254) (layer "F.Cu") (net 11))
 (segment (start 32.131 163.3695) (end 32.075 163.4255) (width 0.254) (layer "F.Cu") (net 11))
 (via (at 32.131 162.179) (size 0.6096) (drill 0.3048) (layers "F.Cu" "B.Cu") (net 11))
 (via (at 30.099 104.013) (size 0.6096) (drill 0.3048) (layers "F.Cu" "B.Cu") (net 11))
 (segment (start 27.432 140.589) (end 31.877 136.144) (width 0.254) (layer "B.Cu") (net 11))
 (segment (start 31.877 136.144) (end 31.877 105.791) (width 0.254) (layer "B.Cu") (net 11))
 (segment (start 31.877 105.791) (end 30.099 104.013) (width 0.254) (layer "B.Cu") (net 11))
 (segment (start 32.131 153.797) (end 27.432 149.098) (width 0.254) (layer "B.Cu") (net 11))
 (segment (start 27.432 149.098) (end 27.432 140.589) (width 0.254) (layer "B.Cu") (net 11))
 (segment (start 32.131 162.179) (end 32.131 153.797) (width 0.254) (layer "B.Cu") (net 11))
 (segment (start 35.56 162.56) (end 35.56 163.4255) (width 0.254) (layer "F.Cu") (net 6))
 (segment (start 31.3205 101.473) (end 31.3205 99.4895) (width 0.254) (layer "F.Cu") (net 6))
 (segment (start 33.782 162.179) (end 35.179 162.179) (width 0.254) (layer "F.Cu") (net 6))
 (segment (start 35.179 162.179) (end 35.56 162.56) (width 0.254) (layer "F.Cu") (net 6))
 (segment (start 31.3205 99.4895) (end 31.369 99.441) (width 0.254) (layer "F.Cu") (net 6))
 (via (at 33.782 162.179) (size 0.6096) (drill 0.3048) (layers "F.Cu" "B.Cu") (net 6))
 (via (at 31.369 99.441) (size 0.6096) (drill 0.3048) (layers "F.Cu" "B.Cu") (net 6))
 (segment (start 28.067 140.843) (end 32.385 136.525) (width 0.254) (layer "B.Cu") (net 6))
 (segment (start 33.02 161.417) (end 33.02 153.67) (width 0.254) (layer "B.Cu") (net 6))
 (segment (start 32.385 136.525) (end 32.385 100.457) (width 0.254) (layer "B.Cu") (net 6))
 (segment (start 33.782 162.179) (end 33.02 161.417) (width 0.254) (layer "B.Cu") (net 6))
 (segment (start 32.385 100.457) (end 31.369 99.441) (width 0.254) (layer "B.Cu") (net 6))
 (segment (start 33.02 153.67) (end 28.067 148.717) (width 0.254) (layer "B.Cu") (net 6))
 (segment (start 28.067 148.717) (end 28.067 140.843) (width 0.254) (layer "B.Cu") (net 6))
 (segment (start 31.633 155.204) (end 29.845 153.416) (width 0.254) (layer "F.Cu") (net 10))
 (segment (start 31.633 156.085) (end 31.633 155.204) (width 0.254) (layer "F.Cu") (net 10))
 (segment (start 29.845 153.416) (end 29.845 152.0425) (width 0.254) (layer "F.Cu") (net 10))
 (segment (start 34.925 152.908) (end 34.925 152.0425) (width 0.254) (layer "F.Cu") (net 14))
 (segment (start 32.883 156.085) (end 32.883 154.95) (width 0.254) (layer "F.Cu") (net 14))
 (segment (start 32.883 154.95) (end 34.925 152.908) (width 0.254) (layer "F.Cu") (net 14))
 (segment (start 33.274 151.13) (end 32.385 152.019) (width 0.254) (layer "F.Cu") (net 9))
 (segment (start 34.133 156.085) (end 36.449 153.769) (width 0.254) (layer "F.Cu") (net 9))
 (segment (start 35.814 151.13) (end 33.274 151.13) (width 0.254) (layer "F.Cu") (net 9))
 (segment (start 32.385 152.019) (end 32.385 152.0425) (width 0.254) (layer "F.Cu") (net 9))
 (segment (start 36.449 151.765) (end 35.814 151.13) (width 0.254) (layer "F.Cu") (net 9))
 (segment (start 36.449 153.769) (end 36.449 151.765) (width 0.254) (layer "F.Cu") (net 9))
 (segment (start 29.535 166.441) (end 29.535 165.2505) (width 0.254) (layer "F.Cu") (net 3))
 (segment (start 31.633 168.539) (end 29.535 166.441) (width 0.254) (layer "F.Cu") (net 3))
 (segment (start 31.633 169.672) (end 31.633 168.539) (width 0.254) (layer "F.Cu") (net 3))
 (segment (start 32.883 168.793) (end 35.56 166.116) (width 0.254) (layer "F.Cu") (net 4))
 (segment (start 32.883 169.672) (end 32.883 168.793) (width 0.254) (layer "F.Cu") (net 4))
 (segment (start 35.56 166.116) (end 35.56 165.2505) (width 0.254) (layer "F.Cu") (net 4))
 (segment (start 34.036 164.338) (end 36.449 164.338) (width 0.254) (layer "F.Cu") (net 5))
 (segment (start 36.957 165.862) (end 34.133 168.686) (width 0.254) (layer "F.Cu") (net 5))
 (segment (start 36.449 164.338) (end 36.957 164.846) (width 0.254) (layer "F.Cu") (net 5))
 (segment (start 32.075 165.2505) (end 33.1235 165.2505) (width 0.254) (layer "F.Cu") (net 5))
 (segment (start 36.957 164.846) (end 36.957 165.862) (width 0.254) (layer "F.Cu") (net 5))
 (segment (start 33.1235 165.2505) (end 34.036 164.338) (width 0.254) (layer "F.Cu") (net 5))
 (segment (start 34.133 168.686) (end 34.133 169.672) (width 0.254) (layer "F.Cu") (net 5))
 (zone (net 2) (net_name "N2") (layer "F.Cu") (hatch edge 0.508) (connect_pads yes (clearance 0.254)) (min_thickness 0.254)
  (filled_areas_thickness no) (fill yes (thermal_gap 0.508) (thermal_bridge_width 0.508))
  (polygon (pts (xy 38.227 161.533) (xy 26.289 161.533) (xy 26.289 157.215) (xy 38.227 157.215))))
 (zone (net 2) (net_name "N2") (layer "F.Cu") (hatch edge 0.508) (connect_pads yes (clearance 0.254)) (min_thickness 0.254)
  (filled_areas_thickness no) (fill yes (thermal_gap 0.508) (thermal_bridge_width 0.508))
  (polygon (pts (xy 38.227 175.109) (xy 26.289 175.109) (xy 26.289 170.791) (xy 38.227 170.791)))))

